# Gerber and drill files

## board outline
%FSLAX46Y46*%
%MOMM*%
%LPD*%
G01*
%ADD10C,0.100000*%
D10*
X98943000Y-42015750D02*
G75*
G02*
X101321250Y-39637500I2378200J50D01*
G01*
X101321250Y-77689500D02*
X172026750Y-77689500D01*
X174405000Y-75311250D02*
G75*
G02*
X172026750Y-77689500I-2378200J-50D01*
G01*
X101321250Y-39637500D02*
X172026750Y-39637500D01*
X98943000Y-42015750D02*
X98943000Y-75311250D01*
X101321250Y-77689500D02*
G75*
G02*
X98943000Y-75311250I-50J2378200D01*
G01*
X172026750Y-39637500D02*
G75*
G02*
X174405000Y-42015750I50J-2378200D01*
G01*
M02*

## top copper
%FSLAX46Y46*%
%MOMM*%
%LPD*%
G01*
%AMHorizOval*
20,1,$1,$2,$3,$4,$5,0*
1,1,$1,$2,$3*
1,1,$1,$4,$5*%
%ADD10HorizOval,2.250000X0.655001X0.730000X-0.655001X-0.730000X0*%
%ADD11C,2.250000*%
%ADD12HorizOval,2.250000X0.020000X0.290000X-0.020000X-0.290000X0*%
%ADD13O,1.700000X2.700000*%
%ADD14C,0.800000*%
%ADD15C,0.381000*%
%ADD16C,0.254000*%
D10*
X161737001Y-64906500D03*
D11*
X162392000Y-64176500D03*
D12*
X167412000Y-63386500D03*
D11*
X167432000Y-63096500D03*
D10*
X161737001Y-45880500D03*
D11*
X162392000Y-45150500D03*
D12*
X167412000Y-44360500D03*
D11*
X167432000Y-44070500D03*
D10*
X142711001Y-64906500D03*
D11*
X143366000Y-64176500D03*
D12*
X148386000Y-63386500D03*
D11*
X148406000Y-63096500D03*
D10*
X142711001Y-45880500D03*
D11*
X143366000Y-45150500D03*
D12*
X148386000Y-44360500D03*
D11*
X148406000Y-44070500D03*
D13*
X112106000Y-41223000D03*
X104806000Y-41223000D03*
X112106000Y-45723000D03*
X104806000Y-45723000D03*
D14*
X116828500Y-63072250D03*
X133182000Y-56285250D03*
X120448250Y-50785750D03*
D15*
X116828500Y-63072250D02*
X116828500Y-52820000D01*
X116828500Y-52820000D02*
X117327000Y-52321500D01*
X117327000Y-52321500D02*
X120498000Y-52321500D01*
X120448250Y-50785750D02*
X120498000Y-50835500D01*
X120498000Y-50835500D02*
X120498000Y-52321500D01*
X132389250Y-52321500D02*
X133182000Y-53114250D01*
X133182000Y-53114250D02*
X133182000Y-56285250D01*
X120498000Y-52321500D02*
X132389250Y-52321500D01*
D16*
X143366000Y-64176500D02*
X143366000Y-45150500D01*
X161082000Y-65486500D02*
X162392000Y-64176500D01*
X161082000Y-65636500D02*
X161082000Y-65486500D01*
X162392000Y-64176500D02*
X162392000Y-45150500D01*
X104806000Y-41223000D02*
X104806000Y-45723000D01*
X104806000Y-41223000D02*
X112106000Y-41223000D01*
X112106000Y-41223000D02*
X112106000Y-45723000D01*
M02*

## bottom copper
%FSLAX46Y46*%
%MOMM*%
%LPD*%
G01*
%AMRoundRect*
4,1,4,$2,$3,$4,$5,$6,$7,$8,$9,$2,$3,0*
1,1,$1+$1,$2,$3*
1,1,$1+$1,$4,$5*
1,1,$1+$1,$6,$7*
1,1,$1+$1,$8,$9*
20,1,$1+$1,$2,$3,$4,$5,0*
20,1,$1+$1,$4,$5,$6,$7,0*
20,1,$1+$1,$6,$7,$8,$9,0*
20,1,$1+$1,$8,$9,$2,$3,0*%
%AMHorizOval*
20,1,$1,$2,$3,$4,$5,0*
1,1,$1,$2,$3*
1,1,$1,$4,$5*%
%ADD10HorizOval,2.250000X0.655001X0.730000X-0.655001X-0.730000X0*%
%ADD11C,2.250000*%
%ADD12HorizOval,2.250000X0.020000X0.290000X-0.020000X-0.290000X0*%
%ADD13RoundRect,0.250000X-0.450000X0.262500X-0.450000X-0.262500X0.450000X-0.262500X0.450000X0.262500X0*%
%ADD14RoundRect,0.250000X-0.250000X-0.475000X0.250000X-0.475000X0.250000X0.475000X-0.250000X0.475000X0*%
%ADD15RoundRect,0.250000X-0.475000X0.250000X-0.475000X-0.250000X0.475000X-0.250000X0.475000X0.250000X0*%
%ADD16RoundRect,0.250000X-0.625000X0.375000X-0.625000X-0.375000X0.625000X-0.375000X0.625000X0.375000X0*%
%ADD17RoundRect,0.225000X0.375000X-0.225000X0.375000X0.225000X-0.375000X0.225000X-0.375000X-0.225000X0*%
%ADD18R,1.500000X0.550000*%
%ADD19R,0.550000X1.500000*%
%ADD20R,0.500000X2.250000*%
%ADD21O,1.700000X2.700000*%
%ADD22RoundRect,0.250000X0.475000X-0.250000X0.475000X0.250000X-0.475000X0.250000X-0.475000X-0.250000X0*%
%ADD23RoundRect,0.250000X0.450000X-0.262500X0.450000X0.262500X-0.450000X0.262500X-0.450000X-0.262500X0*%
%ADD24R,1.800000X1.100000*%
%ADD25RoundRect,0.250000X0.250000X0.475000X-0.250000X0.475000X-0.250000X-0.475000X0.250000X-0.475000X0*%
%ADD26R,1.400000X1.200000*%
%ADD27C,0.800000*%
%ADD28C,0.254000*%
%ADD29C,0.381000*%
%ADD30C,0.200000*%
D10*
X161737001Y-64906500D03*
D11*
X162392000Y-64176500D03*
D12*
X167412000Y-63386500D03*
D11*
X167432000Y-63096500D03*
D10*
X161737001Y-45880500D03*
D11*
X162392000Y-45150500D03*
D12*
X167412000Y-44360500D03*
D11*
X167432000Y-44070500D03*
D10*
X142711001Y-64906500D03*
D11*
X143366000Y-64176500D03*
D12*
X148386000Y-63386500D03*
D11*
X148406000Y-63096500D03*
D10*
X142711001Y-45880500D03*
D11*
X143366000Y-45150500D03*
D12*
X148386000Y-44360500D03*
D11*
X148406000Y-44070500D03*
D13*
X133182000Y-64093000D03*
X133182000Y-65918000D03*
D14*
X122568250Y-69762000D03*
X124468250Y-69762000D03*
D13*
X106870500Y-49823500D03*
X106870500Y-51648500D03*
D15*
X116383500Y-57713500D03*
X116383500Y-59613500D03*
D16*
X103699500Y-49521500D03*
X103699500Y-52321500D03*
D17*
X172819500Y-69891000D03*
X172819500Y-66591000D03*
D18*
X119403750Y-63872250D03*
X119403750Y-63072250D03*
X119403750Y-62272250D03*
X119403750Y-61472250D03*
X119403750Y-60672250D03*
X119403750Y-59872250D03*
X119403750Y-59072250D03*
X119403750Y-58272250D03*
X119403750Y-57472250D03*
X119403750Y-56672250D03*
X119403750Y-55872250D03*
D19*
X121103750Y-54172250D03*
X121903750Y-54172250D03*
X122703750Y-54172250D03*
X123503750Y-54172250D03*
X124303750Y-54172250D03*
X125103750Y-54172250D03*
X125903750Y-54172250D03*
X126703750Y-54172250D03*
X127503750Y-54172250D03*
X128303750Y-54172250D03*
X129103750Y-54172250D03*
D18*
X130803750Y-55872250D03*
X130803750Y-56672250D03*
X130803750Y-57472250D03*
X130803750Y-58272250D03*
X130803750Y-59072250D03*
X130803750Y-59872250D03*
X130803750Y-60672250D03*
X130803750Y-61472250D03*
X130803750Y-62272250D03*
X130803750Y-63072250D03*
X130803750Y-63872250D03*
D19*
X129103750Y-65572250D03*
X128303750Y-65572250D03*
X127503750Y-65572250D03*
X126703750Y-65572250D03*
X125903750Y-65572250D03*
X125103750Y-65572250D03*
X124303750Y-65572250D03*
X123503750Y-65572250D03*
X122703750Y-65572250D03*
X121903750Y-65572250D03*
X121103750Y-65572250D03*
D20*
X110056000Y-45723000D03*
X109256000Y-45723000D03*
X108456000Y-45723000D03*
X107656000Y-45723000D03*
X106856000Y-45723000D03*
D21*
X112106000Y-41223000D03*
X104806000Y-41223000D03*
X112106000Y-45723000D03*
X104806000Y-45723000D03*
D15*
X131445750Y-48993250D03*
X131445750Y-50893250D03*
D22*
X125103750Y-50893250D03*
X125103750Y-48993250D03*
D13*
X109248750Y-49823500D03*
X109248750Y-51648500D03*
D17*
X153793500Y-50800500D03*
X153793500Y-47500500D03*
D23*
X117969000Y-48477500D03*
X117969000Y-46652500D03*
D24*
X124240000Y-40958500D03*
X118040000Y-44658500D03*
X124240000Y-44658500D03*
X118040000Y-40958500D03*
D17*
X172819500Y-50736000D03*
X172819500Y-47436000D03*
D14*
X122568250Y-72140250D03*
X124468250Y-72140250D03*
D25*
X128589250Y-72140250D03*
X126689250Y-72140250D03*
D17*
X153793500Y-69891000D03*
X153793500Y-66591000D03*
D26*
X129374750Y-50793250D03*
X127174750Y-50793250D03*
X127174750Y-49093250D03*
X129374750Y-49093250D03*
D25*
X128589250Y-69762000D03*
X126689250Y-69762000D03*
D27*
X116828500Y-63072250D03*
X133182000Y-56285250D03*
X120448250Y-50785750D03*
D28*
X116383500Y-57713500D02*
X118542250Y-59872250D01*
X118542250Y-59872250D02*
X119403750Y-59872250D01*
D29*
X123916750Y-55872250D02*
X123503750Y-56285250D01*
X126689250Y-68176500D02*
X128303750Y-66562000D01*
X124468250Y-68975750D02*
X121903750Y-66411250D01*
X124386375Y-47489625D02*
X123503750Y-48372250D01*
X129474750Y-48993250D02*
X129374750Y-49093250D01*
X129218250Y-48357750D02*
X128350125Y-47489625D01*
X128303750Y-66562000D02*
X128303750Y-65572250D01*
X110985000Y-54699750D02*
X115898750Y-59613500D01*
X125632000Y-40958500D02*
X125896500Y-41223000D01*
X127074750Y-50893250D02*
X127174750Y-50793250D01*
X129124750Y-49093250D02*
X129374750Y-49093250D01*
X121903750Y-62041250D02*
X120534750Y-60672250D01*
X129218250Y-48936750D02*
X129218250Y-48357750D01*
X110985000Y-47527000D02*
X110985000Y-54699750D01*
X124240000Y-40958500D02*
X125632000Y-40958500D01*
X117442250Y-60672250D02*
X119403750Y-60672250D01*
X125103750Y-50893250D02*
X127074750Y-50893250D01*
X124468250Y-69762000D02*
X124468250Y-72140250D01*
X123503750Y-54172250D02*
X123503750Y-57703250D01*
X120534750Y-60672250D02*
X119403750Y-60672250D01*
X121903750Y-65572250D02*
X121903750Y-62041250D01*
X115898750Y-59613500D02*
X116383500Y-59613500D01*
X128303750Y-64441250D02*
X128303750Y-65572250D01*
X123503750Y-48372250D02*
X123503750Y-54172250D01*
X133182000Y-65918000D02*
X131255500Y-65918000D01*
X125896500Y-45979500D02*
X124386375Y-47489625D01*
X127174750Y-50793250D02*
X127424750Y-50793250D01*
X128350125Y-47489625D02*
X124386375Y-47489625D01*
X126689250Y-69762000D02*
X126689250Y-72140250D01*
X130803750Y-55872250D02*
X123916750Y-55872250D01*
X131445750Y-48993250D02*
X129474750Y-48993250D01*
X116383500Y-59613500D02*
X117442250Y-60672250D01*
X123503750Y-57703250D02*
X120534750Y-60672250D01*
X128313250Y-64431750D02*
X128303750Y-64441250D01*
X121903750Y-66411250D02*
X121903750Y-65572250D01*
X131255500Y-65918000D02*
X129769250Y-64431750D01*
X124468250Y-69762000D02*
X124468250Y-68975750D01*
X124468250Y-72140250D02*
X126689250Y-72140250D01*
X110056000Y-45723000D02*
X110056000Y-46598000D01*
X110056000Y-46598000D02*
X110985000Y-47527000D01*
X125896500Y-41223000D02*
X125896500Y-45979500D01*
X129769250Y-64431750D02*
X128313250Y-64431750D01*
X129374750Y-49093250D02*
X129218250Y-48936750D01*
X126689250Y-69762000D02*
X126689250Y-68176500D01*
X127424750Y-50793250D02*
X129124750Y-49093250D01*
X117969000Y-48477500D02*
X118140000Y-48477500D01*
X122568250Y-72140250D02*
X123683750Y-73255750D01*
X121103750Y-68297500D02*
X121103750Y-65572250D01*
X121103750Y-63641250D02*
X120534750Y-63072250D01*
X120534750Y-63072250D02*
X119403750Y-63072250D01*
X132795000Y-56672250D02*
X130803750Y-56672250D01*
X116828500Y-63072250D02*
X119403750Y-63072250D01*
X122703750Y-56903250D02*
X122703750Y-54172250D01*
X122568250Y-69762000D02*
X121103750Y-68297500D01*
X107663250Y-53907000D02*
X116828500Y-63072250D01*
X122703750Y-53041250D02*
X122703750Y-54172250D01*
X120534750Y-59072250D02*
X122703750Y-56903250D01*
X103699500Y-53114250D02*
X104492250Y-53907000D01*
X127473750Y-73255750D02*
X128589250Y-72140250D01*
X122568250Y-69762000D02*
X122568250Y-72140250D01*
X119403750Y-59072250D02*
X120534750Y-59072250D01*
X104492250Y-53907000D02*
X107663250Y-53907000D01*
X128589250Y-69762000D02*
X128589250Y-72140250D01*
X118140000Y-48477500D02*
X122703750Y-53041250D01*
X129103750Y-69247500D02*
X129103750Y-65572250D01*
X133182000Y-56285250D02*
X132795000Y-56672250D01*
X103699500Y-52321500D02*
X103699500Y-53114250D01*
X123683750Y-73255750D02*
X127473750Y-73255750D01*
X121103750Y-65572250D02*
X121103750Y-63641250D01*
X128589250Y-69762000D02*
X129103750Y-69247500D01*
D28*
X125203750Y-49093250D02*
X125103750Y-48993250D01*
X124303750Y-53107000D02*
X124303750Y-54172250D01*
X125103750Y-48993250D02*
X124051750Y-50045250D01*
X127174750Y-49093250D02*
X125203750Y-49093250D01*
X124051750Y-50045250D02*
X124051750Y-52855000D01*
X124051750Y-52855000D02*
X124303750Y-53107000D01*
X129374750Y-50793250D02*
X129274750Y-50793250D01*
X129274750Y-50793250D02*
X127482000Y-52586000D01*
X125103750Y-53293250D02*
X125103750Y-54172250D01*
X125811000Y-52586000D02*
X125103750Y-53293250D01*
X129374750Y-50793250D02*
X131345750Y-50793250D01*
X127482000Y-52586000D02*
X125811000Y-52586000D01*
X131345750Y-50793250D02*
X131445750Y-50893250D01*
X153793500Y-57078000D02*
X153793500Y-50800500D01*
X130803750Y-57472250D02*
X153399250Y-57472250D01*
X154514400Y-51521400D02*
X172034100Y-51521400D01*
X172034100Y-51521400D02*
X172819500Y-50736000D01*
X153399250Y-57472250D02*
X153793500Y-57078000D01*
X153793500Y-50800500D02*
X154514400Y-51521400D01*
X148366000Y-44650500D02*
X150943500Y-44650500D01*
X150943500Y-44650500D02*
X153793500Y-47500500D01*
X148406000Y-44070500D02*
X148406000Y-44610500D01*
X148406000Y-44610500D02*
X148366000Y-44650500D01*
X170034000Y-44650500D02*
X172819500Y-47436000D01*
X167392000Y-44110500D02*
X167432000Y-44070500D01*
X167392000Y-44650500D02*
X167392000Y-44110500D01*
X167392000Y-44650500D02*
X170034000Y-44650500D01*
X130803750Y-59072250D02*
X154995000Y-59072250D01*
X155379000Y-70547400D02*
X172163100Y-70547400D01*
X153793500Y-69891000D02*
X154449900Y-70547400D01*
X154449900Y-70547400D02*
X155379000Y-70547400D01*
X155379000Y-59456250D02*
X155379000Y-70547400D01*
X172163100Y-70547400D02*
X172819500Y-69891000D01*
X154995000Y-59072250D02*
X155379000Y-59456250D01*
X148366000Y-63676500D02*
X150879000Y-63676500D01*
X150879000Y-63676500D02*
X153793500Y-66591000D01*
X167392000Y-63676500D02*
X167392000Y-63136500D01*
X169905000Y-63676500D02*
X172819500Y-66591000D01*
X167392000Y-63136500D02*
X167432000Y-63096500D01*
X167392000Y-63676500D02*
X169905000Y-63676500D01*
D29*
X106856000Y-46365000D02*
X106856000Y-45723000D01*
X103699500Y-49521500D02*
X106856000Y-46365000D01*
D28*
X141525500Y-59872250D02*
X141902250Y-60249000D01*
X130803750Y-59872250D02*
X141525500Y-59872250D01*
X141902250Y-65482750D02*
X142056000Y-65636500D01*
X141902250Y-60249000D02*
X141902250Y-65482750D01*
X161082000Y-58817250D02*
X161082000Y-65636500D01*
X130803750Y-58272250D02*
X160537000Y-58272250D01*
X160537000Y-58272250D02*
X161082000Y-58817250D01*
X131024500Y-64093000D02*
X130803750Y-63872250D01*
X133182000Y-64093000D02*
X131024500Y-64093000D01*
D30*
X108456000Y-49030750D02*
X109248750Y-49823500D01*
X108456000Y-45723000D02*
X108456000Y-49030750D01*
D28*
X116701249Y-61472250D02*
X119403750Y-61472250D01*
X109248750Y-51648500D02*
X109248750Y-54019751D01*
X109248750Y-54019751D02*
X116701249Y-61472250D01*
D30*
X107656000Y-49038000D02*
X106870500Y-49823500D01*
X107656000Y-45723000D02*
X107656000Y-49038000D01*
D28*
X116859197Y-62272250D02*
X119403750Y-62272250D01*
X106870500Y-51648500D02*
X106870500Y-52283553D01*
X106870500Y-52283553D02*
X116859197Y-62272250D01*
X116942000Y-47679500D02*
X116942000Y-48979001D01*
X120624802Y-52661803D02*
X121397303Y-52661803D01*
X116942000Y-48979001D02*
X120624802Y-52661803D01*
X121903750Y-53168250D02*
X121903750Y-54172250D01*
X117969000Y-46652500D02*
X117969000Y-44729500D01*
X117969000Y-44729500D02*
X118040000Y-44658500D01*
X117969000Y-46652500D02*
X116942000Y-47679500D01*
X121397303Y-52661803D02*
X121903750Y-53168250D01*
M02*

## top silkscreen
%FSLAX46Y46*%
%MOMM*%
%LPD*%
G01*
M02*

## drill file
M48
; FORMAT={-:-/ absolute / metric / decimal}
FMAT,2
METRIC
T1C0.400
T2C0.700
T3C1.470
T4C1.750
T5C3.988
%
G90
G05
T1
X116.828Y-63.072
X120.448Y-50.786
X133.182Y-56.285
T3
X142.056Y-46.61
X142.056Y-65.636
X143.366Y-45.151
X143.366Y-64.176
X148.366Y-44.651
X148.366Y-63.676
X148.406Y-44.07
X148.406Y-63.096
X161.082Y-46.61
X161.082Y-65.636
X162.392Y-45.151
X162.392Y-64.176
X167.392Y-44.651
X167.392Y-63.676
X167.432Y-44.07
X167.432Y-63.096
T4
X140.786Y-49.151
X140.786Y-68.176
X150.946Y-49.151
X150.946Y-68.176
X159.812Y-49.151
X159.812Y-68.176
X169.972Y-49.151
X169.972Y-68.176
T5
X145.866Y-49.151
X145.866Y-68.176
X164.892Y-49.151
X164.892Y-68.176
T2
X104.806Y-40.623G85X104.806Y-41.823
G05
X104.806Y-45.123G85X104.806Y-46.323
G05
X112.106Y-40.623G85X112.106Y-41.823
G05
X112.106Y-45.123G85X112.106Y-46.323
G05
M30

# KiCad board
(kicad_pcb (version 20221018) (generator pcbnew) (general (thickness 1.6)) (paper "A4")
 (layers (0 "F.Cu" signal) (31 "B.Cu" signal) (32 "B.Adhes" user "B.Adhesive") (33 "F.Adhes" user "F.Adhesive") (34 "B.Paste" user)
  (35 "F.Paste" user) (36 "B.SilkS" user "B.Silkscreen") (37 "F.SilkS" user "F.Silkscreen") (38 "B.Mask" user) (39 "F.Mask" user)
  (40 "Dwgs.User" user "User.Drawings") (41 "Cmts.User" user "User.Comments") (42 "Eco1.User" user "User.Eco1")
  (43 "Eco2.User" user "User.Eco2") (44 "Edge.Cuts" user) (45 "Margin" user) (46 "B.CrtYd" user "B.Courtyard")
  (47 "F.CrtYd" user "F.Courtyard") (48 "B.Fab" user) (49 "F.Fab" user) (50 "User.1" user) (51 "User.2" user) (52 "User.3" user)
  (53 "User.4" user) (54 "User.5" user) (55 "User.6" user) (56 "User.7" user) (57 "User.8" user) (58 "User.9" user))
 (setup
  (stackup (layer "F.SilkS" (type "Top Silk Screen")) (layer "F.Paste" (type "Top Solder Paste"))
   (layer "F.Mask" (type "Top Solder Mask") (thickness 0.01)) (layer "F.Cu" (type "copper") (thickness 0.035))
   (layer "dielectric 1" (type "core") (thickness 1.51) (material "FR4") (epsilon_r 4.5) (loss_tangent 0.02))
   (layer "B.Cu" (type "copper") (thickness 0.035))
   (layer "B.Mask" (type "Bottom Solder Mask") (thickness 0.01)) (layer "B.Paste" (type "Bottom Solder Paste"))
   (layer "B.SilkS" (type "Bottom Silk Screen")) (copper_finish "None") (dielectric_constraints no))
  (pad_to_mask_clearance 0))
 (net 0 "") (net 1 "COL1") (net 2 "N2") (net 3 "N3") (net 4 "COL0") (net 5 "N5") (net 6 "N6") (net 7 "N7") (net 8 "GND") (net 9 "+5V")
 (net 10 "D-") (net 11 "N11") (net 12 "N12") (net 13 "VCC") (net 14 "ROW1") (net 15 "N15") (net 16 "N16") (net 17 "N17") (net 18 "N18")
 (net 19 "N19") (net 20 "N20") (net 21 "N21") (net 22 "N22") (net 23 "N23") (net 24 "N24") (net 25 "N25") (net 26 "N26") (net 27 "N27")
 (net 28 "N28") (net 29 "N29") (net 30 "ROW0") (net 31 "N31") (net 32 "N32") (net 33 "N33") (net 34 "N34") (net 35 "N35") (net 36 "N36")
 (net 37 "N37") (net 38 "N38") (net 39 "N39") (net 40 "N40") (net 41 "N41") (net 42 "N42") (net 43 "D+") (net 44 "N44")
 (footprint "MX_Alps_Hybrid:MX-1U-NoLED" (layer "F.Cu") (at 164.892 68.1765)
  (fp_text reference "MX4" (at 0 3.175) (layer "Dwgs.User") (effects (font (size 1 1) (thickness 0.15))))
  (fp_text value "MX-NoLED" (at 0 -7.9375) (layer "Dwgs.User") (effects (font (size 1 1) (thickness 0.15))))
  (pad "" np_thru_hole circle (at -5.08 0 48.0996) (size 1.75 1.75) (drill 1.75) (layers "*.Cu" "*.Mask"))
  (pad "" np_thru_hole circle (at 0 0) (size 3.9878 3.9878) (drill 3.9878) (layers "*.Cu" "*.Mask"))
  (pad "" np_thru_hole circle (at 5.08 0 48.0996) (size 1.75 1.75) (drill 1.75) (layers "*.Cu" "*.Mask"))
  (pad "1" thru_hole oval (at -3.81 -2.54 48.0996) (size 4.211556 2.25) (drill 1.47 (offset 0.980778 0)) (layers "*.Cu" "B.Mask")
   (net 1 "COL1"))
  (pad "1" thru_hole circle (at -2.5 -4) (size 2.25 2.25) (drill 1.47) (layers "*.Cu" "B.Mask") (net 1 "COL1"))
  (pad "2" thru_hole oval (at 2.5 -4.5 86.0548) (size 2.831378 2.25) (drill 1.47 (offset 0.290689 0)) (layers "*.Cu" "B.Mask") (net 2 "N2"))
  (pad "2" thru_hole circle (at 2.54 -5.08) (size 2.25 2.25) (drill 1.47) (layers "*.Cu" "B.Mask") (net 2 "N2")))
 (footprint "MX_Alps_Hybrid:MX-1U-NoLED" (layer "F.Cu") (at 164.892 49.1505)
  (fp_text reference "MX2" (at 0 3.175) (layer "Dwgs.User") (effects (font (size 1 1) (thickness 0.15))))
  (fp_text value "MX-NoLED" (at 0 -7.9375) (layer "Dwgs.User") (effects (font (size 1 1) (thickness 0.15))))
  (pad "" np_thru_hole circle (at -5.08 0 48.0996) (size 1.75 1.75) (drill 1.75) (layers "*.Cu" "*.Mask"))
  (pad "" np_thru_hole circle (at 0 0) (size 3.9878 3.9878) (drill 3.9878) (layers "*.Cu" "*.Mask"))
  (pad "" np_thru_hole circle (at 5.08 0 48.0996) (size 1.75 1.75) (drill 1.75) (layers "*.Cu" "*.Mask"))
  (pad "1" thru_hole oval (at -3.81 -2.54 48.0996) (size 4.211556 2.25) (drill 1.47 (offset 0.980778 0)) (layers "*.Cu" "B.Mask")
   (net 1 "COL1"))
  (pad "1" thru_hole circle (at -2.5 -4) (size 2.25 2.25) (drill 1.47) (layers "*.Cu" "B.Mask") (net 1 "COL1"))
  (pad "2" thru_hole oval (at 2.5 -4.5 86.0548) (size 2.831378 2.25) (drill 1.47 (offset 0.290689 0)) (layers "*.Cu" "B.Mask") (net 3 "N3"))
  (pad "2" thru_hole circle (at 2.54 -5.08) (size 2.25 2.25) (drill 1.47) (layers "*.Cu" "B.Mask") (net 3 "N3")))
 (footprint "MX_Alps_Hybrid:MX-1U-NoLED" (layer "F.Cu") (at 145.866 68.1765)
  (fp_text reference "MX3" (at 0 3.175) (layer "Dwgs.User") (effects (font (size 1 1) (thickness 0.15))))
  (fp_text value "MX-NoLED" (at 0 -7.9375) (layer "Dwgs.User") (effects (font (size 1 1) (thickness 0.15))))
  (pad "" np_thru_hole circle (at -5.08 0 48.0996) (size 1.75 1.75) (drill 1.75) (layers "*.Cu" "*.Mask"))
  (pad "" np_thru_hole circle (at 0 0) (size 3.9878 3.9878) (drill 3.9878) (layers "*.Cu" "*.Mask"))
  (pad "" np_thru_hole circle (at 5.08 0 48.0996) (size 1.75 1.75) (drill 1.75) (layers "*.Cu" "*.Mask"))
  (pad "1" thru_hole oval (at -3.81 -2.54 48.0996) (size 4.211556 2.25) (drill 1.47 (offset 0.980778 0)) (layers "*.Cu" "B.Mask")
   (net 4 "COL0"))
  (pad "1" thru_hole circle (at -2.5 -4) (size 2.25 2.25) (drill 1.47) (layers "*.Cu" "B.Mask") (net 4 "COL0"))
  (pad "2" thru_hole oval (at 2.5 -4.5 86.0548) (size 2.831378 2.25) (drill 1.47 (offset 0.290689 0)) (layers "*.Cu" "B.Mask") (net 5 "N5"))
  (pad "2" thru_hole circle (at 2.54 -5.08) (size 2.25 2.25) (drill 1.47) (layers "*.Cu" "B.Mask") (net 5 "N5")))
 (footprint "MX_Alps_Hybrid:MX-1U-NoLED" (layer "F.Cu") (at 145.866 49.1505)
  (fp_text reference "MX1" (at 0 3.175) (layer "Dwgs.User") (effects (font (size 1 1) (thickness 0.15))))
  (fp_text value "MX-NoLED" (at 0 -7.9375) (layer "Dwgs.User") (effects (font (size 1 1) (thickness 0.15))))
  (pad "" np_thru_hole circle (at -5.08 0 48.0996) (size 1.75 1.75) (drill 1.75) (layers "*.Cu" "*.Mask"))
  (pad "" np_thru_hole circle (at 0 0) (size 3.9878 3.9878) (drill 3.9878) (layers "*.Cu" "*.Mask"))
  (pad "" np_thru_hole circle (at 5.08 0 48.0996) (size 1.75 1.75) (drill 1.75) (layers "*.Cu" "*.Mask"))
  (pad "1" thru_hole oval (at -3.81 -2.54 48.0996) (size 4.211556 2.25) (drill 1.47 (offset 0.980778 0)) (layers "*.Cu" "B.Mask")
   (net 4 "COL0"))
  (pad "1" thru_hole circle (at -2.5 -4) (size 2.25 2.25) (drill 1.47) (layers "*.Cu" "B.Mask") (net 4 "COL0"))
  (pad "2" thru_hole oval (at 2.5 -4.5 86.0548) (size 2.831378 2.25) (drill 1.47 (offset 0.290689 0)) (layers "*.Cu" "B.Mask") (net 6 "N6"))
  (pad "2" thru_hole circle (at 2.54 -5.08) (size 2.25 2.25) (drill 1.47) (layers "*.Cu" "B.Mask") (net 6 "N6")))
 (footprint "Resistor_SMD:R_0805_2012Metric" (layer "B.Cu") (at 133.182 65.0055 -90)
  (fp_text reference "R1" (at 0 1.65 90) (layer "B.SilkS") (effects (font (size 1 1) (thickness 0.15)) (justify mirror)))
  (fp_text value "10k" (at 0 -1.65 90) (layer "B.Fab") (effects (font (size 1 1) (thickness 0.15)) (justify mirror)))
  (pad "1" smd roundrect (at -0.9125 0 270) (size 1.025 1.4) (layers "B.Cu" "B.Paste" "B.Mask") (roundrect_rratio 0.243902) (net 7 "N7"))
  (pad "2" smd roundrect (at 0.9125 0 270) (size 1.025 1.4) (layers "B.Cu" "B.Paste" "B.Mask") (roundrect_rratio 0.243902) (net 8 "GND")))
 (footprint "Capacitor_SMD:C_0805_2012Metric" (layer "B.Cu") (at 123.51825 69.762)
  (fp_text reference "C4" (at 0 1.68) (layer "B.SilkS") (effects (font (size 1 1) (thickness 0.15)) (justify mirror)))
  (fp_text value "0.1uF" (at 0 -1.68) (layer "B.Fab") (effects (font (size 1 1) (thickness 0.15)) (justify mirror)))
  (pad "1" smd roundrect (at -0.95 0) (size 1 1.45) (layers "B.Cu" "B.Paste" "B.Mask") (roundrect_rratio 0.25) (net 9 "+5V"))
  (pad "2" smd roundrect (at 0.95 0) (size 1 1.45) (layers "B.Cu" "B.Paste" "B.Mask") (roundrect_rratio 0.25) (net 8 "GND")))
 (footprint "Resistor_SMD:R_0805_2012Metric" (layer "B.Cu") (at 106.8705 50.736 -90)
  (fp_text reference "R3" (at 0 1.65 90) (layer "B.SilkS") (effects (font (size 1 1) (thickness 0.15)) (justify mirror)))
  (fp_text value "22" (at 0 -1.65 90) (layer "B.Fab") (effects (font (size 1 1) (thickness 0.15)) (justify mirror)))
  (pad "1" smd roundrect (at -0.9125 0 270) (size 1.025 1.4) (layers "B.Cu" "B.Paste" "B.Mask") (roundrect_rratio 0.243902) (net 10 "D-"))
  (pad "2" smd roundrect (at 0.9125 0 270) (size 1.025 1.4) (layers "B.Cu" "B.Paste" "B.Mask") (roundrect_rratio 0.243902) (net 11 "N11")))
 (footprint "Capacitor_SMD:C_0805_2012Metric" (layer "B.Cu") (at 116.3835 58.6635 -90)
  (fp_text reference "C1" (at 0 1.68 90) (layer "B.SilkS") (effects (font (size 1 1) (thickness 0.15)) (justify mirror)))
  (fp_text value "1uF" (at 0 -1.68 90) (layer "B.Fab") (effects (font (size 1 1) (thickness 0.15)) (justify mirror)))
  (pad "1" smd roundrect (at -0.95 0 270) (size 1 1.45) (layers "B.Cu" "B.Paste" "B.Mask") (roundrect_rratio 0.25) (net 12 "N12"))
  (pad "2" smd roundrect (at 0.95 0 270) (size 1 1.45) (layers "B.Cu" "B.Paste" "B.Mask") (roundrect_rratio 0.25) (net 8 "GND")))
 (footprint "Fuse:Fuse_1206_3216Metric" (layer "B.Cu") (at 103.6995 50.9215 -90)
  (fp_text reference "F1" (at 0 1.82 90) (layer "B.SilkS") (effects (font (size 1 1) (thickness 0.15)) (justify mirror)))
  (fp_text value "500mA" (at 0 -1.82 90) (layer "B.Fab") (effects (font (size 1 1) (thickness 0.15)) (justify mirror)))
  (pad "1" smd roundrect (at -1.4 0 270) (size 1.25 1.75) (layers "B.Cu" "B.Paste" "B.Mask") (roundrect_rratio 0.2) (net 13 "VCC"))
  (pad "2" smd roundrect (at 1.4 0 270) (size 1.25 1.75) (layers "B.Cu" "B.Paste" "B.Mask") (roundrect_rratio 0.2) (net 9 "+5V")))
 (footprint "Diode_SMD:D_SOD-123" (layer "B.Cu") (at 172.8195 68.241 90)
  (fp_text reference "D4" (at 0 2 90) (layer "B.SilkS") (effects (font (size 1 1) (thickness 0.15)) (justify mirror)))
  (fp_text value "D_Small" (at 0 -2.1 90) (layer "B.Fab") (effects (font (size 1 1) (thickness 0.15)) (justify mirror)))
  (pad "1" smd roundrect (at -1.65 0 90) (size 0.9 1.2) (layers "B.Cu" "B.Paste" "B.Mask") (roundrect_rratio 0.25) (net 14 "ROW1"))
  (pad "2" smd roundrect (at 1.65 0 90) (size 0.9 1.2) (layers "B.Cu" "B.Paste" "B.Mask") (roundrect_rratio 0.25) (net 2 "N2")))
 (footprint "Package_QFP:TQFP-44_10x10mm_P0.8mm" (layer "B.Cu") (at 125.10375 59.87225)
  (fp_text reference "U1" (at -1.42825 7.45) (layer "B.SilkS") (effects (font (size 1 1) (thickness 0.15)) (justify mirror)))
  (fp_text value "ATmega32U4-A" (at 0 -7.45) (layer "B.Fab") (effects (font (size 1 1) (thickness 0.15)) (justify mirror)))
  (pad "1" smd rect (at -5.7 4) (size 1.5 0.55) (layers "B.Cu" "B.Paste" "B.Mask") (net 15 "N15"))
  (pad "2" smd rect (at -5.7 3.2) (size 1.5 0.55) (layers "B.Cu" "B.Paste" "B.Mask") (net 9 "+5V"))
  (pad "3" smd rect (at -5.7 2.4) (size 1.5 0.55) (layers "B.Cu" "B.Paste" "B.Mask") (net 11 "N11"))
  (pad "4" smd rect (at -5.7 1.6) (size 1.5 0.55) (layers "B.Cu" "B.Paste" "B.Mask") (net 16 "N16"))
  (pad "5" smd rect (at -5.7 0.8) (size 1.5 0.55) (layers "B.Cu" "B.Paste" "B.Mask") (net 8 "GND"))
  (pad "6" smd rect (at -5.7 0) (size 1.5 0.55) (layers "B.Cu" "B.Paste" "B.Mask") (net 12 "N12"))
  (pad "7" smd rect (at -5.7 -0.8) (size 1.5 0.55) (layers "B.Cu" "B.Paste" "B.Mask") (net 9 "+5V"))
  (pad "8" smd rect (at -5.7 -1.6) (size 1.5 0.55) (layers "B.Cu" "B.Paste" "B.Mask") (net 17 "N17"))
  (pad "9" smd rect (at -5.7 -2.4) (size 1.5 0.55) (layers "B.Cu" "B.Paste" "B.Mask") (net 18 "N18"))
  (pad "10" smd rect (at -5.7 -3.2) (size 1.5 0.55) (layers "B.Cu" "B.Paste" "B.Mask") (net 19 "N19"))
  (pad "11" smd rect (at -5.7 -4) (size 1.5 0.55) (layers "B.Cu" "B.Paste" "B.Mask") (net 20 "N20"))
  (pad "12" smd rect (at -4 -5.7 270) (size 1.5 0.55) (layers "B.Cu" "B.Paste" "B.Mask") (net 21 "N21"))
  (pad "13" smd rect (at -3.2 -5.7 270) (size 1.5 0.55) (layers "B.Cu" "B.Paste" "B.Mask") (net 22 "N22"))
  (pad "14" smd rect (at -2.4 -5.7 270) (size 1.5 0.55) (layers "B.Cu" "B.Paste" "B.Mask") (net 9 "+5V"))
  (pad "15" smd rect (at -1.6 -5.7 270) (size 1.5 0.55) (layers "B.Cu" "B.Paste" "B.Mask") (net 8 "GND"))
  (pad "16" smd rect (at -0.8 -5.7 270) (size 1.5 0.55) (layers "B.Cu" "B.Paste" "B.Mask") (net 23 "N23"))
  (pad "17" smd rect (at 0 -5.7 270) (size 1.5 0.55) (layers "B.Cu" "B.Paste" "B.Mask") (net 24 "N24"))
  (pad "18" smd rect (at 0.8 -5.7 270) (size 1.5 0.55) (layers "B.Cu" "B.Paste" "B.Mask") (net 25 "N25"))
  (pad "19" smd rect (at 1.6 -5.7 270) (size 1.5 0.55) (layers "B.Cu" "B.Paste" "B.Mask") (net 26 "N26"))
  (pad "20" smd rect (at 2.4 -5.7 270) (size 1.5 0.55) (layers "B.Cu" "B.Paste" "B.Mask") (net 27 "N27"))
  (pad "21" smd rect (at 3.2 -5.7 270) (size 1.5 0.55) (layers "B.Cu" "B.Paste" "B.Mask") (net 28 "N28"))
  (pad "22" smd rect (at 4 -5.7 270) (size 1.5 0.55) (layers "B.Cu" "B.Paste" "B.Mask") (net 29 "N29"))
  (pad "23" smd rect (at 5.7 -4) (size 1.5 0.55) (layers "B.Cu" "B.Paste" "B.Mask") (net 8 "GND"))
  (pad "24" smd rect (at 5.7 -3.2) (size 1.5 0.55) (layers "B.Cu" "B.Paste" "B.Mask") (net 9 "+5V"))
  (pad "25" smd rect (at 5.7 -2.4) (size 1.5 0.55) (layers "B.Cu" "B.Paste" "B.Mask") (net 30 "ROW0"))
  (pad "26" smd rect (at 5.7 -1.6) (size 1.5 0.55) (layers "B.Cu" "B.Paste" "B.Mask") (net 1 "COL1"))
  (pad "27" smd rect (at 5.7 -0.8) (size 1.5 0.55) (layers "B.Cu" "B.Paste" "B.Mask") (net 14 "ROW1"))
  (pad "28" smd rect (at 5.7 0) (size 1.5 0.55) (layers "B.Cu" "B.Paste" "B.Mask") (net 4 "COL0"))
  (pad "29" smd rect (at 5.7 0.8) (size 1.5 0.55) (layers "B.Cu" "B.Paste" "B.Mask") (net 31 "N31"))
  (pad "30" smd rect (at 5.7 1.6) (size 1.5 0.55) (layers "B.Cu" "B.Paste" "B.Mask") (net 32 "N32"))
  (pad "31" smd rect (at 5.7 2.4) (size 1.5 0.55) (layers "B.Cu" "B.Paste" "B.Mask") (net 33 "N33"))
  (pad "32" smd rect (at 5.7 3.2) (size 1.5 0.55) (layers "B.Cu" "B.Paste" "B.Mask") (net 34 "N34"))
  (pad "33" smd rect (at 5.7 4) (size 1.5 0.55) (layers "B.Cu" "B.Paste" "B.Mask") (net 7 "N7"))
  (pad "34" smd rect (at 4 5.7 270) (size 1.5 0.55) (layers "B.Cu" "B.Paste" "B.Mask") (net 9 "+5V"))
  (pad "35" smd rect (at 3.2 5.7 270) (size 1.5 0.55) (layers "B.Cu" "B.Paste" "B.Mask") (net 8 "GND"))
  (pad "36" smd rect (at 2.4 5.7 270) (size 1.5 0.55) (layers "B.Cu" "B.Paste" "B.Mask") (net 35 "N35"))
  (pad "37" smd rect (at 1.6 5.7 270) (size 1.5 0.55) (layers "B.Cu" "B.Paste" "B.Mask") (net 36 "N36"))
  (pad "38" smd rect (at 0.8 5.7 270) (size 1.5 0.55) (layers "B.Cu" "B.Paste" "B.Mask") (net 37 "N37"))
  (pad "39" smd rect (at 0 5.7 270) (size 1.5 0.55) (layers "B.Cu" "B.Paste" "B.Mask") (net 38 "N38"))
  (pad "40" smd rect (at -0.8 5.7 270) (size 1.5 0.55) (layers "B.Cu" "B.Paste" "B.Mask") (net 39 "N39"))
  (pad "41" smd rect (at -1.6 5.7 270) (size 1.5 0.55) (layers "B.Cu" "B.Paste" "B.Mask") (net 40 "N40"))
  (pad "42" smd rect (at -2.4 5.7 270) (size 1.5 0.55) (layers "B.Cu" "B.Paste" "B.Mask") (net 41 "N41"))
  (pad "43" smd rect (at -3.2 5.7 270) (size 1.5 0.55) (layers "B.Cu" "B.Paste" "B.Mask") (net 8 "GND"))
  (pad "44" smd rect (at -4 5.7 270) (size 1.5 0.55) (layers "B.Cu" "B.Paste" "B.Mask") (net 9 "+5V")))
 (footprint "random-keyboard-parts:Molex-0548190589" (layer "B.Cu") (at 108.456 41.223 -90)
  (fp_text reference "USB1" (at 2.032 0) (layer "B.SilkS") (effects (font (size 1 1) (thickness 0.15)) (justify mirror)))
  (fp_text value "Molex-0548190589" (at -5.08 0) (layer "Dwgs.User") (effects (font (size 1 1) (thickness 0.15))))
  (pad "1" smd rect (at 4.5 -1.6 270) (size 2.25 0.5) (layers "B.Cu" "B.Paste" "B.Mask") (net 8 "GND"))
  (pad "2" smd rect (at 4.5 -0.8 270) (size 2.25 0.5) (layers "B.Cu" "B.Paste" "B.Mask") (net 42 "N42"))
  (pad "3" smd rect (at 4.5 0 270) (size 2.25 0.5) (layers "B.Cu" "B.Paste" "B.Mask") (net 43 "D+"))
  (pad "4" smd rect (at 4.5 0.8 270) (size 2.25 0.5) (layers "B.Cu" "B.Paste" "B.Mask") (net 10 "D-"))
  (pad "5" smd rect (at 4.5 1.6 270) (size 2.25 0.5) (layers "B.Cu" "B.Paste" "B.Mask") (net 13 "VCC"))
  (pad "6" thru_hole oval (at 0 -3.65 270) (size 2.7 1.7) (drill oval 1.9 0.7) (layers "*.Cu" "*.Mask") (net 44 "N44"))
  (pad "6" thru_hole oval (at 0 3.65 270) (size 2.7 1.7) (drill oval 1.9 0.7) (layers "*.Cu" "*.Mask") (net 44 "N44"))
  (pad "6" thru_hole oval (at 4.5 -3.65 270) (size 2.7 1.7) (drill oval 1.9 0.7) (layers "*.Cu" "*.Mask") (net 44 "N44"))
  (pad "6" thru_hole oval (at 4.5 3.65 270) (size 2.7 1.7) (drill oval 1.9 0.7) (layers "*.Cu" "*.Mask") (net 44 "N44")))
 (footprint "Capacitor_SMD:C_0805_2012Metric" (layer "B.Cu") (at 131.44575 49.94325 -90)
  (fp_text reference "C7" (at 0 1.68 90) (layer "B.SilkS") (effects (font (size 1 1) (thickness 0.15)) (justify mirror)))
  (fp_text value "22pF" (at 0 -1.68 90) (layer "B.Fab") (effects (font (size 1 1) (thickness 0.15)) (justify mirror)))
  (pad "1" smd roundrect (at -0.95 0 270) (size 1 1.45) (layers "B.Cu" "B.Paste" "B.Mask") (roundrect_rratio 0.25) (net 8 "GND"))
  (pad "2" smd roundrect (at 0.95 0 270) (size 1 1.45) (layers "B.Cu" "B.Paste" "B.Mask") (roundrect_rratio 0.25) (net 24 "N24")))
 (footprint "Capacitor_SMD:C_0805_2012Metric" (layer "B.Cu") (at 125.10375 49.94325 90)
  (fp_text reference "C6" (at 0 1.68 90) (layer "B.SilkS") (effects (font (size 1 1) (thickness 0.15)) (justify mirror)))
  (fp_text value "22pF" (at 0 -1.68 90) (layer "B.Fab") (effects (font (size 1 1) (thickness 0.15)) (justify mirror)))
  (pad "1" smd roundrect (at -0.95 0 90) (size 1 1.45) (layers "B.Cu" "B.Paste" "B.Mask") (roundrect_rratio 0.25) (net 8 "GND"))
  (pad "2" smd roundrect (at 0.95 0 90) (size 1 1.45) (layers "B.Cu" "B.Paste" "B.Mask") (roundrect_rratio 0.25) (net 23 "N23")))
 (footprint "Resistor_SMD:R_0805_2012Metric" (layer "B.Cu") (at 109.24875 50.736 -90)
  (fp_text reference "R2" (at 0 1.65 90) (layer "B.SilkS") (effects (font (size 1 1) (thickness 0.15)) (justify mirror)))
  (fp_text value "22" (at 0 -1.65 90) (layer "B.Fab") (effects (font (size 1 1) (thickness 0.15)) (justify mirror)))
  (pad "1" smd roundrect (at -0.9125 0 270) (size 1.025 1.4) (layers "B.Cu" "B.Paste" "B.Mask") (roundrect_rratio 0.243902) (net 43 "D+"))
  (pad "2" smd roundrect (at 0.9125 0 270) (size 1.025 1.4) (layers "B.Cu" "B.Paste" "B.Mask") (roundrect_rratio 0.243902) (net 16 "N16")))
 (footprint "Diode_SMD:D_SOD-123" (layer "B.Cu") (at 153.7935 49.1505 90)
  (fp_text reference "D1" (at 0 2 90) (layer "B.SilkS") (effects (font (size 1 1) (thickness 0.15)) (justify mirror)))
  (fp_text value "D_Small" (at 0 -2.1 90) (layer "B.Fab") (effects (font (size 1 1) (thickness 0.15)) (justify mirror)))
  (pad "1" smd roundrect (at -1.65 0 90) (size 0.9 1.2) (layers "B.Cu" "B.Paste" "B.Mask") (roundrect_rratio 0.25) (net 30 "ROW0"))
  (pad "2" smd roundrect (at 1.65 0 90) (size 0.9 1.2) (layers "B.Cu" "B.Paste" "B.Mask") (roundrect_rratio 0.25) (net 6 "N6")))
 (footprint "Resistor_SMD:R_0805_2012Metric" (layer "B.Cu") (at 117.969 47.565 90)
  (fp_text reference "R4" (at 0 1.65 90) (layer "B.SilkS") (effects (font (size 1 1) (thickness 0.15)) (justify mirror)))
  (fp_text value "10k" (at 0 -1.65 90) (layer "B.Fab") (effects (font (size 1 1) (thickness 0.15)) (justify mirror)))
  (pad "1" smd roundrect (at -0.9125 0 90) (size 1.025 1.4) (layers "B.Cu" "B.Paste" "B.Mask") (roundrect_rratio 0.243902) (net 9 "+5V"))
  (pad "2" smd roundrect (at 0.9125 0 90) (size 1.025 1.4) (layers "B.Cu" "B.Paste" "B.Mask") (roundrect_rratio 0.243902) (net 22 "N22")))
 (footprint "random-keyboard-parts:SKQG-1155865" (layer "B.Cu") (at 121.14 42.8085)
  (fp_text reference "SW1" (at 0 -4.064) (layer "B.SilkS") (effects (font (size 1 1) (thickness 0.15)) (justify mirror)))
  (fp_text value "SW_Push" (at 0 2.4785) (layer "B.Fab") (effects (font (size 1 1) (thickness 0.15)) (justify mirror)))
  (pad "1" smd rect (at 3.1 -1.85) (size 1.8 1.1) (layers "B.Cu" "B.Paste" "B.Mask") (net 8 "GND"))
  (pad "2" smd rect (at -3.1 1.85) (size 1.8 1.1) (layers "B.Cu" "B.Paste" "B.Mask") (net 22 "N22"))
  (pad "3" smd rect (at 3.1 1.85) (size 1.8 1.1) (layers "B.Cu" "B.Paste" "B.Mask"))
  (pad "4" smd rect (at -3.1 -1.85) (size 1.8 1.1) (layers "B.Cu" "B.Paste" "B.Mask")))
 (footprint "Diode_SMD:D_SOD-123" (layer "B.Cu") (at 172.8195 49.086 90)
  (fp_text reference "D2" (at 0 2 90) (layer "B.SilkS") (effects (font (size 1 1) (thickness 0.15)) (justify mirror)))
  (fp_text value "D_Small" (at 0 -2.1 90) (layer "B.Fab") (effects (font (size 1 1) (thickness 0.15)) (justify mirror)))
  (pad "1" smd roundrect (at -1.65 0 90) (size 0.9 1.2) (layers "B.Cu" "B.Paste" "B.Mask") (roundrect_rratio 0.25) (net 30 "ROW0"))
  (pad "2" smd roundrect (at 1.65 0 90) (size 0.9 1.2) (layers "B.Cu" "B.Paste" "B.Mask") (roundrect_rratio 0.25) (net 3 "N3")))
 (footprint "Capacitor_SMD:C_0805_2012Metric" (layer "B.Cu") (at 123.51825 72.14025)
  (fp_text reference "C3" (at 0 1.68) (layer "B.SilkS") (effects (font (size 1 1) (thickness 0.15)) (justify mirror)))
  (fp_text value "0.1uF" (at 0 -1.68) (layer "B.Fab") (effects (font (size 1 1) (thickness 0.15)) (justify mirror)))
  (pad "1" smd roundrect (at -0.95 0) (size 1 1.45) (layers "B.Cu" "B.Paste" "B.Mask") (roundrect_rratio 0.25) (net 9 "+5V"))
  (pad "2" smd roundrect (at 0.95 0) (size 1 1.45) (layers "B.Cu" "B.Paste" "B.Mask") (roundrect_rratio 0.25) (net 8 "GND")))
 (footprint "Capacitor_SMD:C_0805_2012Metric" (layer "B.Cu") (at 127.63925 72.14025 180)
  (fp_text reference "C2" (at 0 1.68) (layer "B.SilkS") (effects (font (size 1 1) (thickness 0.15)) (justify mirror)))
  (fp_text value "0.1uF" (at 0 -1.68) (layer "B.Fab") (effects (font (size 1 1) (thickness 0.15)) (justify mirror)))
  (pad "1" smd roundrect (at -0.95 0 180) (size 1 1.45) (layers "B.Cu" "B.Paste" "B.Mask") (roundrect_rratio 0.25) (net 9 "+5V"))
  (pad "2" smd roundrect (at 0.95 0 180) (size 1 1.45) (layers "B.Cu" "B.Paste" "B.Mask") (roundrect_rratio 0.25) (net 8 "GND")))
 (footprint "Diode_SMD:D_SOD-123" (layer "B.Cu") (at 153.7935 68.241 90)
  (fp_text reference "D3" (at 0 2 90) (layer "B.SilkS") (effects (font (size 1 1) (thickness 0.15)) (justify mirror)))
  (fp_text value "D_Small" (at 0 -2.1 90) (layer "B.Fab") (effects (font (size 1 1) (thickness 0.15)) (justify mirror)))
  (pad "1" smd roundrect (at -1.65 0 90) (size 0.9 1.2) (layers "B.Cu" "B.Paste" "B.Mask") (roundrect_rratio 0.25) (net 14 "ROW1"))
  (pad "2" smd roundrect (at 1.65 0 90) (size 0.9 1.2) (layers "B.Cu" "B.Paste" "B.Mask") (roundrect_rratio 0.25) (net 5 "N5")))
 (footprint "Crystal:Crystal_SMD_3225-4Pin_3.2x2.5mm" (layer "B.Cu") (at 128.27475 49.94325 180)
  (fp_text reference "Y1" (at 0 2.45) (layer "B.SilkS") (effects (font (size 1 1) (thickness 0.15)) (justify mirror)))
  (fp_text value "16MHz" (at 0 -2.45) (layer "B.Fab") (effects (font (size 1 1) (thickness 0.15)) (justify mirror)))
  (pad "1" smd rect (at -1.1 -0.85 180) (size 1.4 1.2) (layers "B.Cu" "B.Paste" "B.Mask") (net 24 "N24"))
  (pad "2" smd rect (at 1.1 -0.85 180) (size 1.4 1.2) (layers "B.Cu" "B.Paste" "B.Mask") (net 8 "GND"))
  (pad "3" smd rect (at 1.1 0.85 180) (size 1.4 1.2) (layers "B.Cu" "B.Paste" "B.Mask") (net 23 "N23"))
  (pad "4" smd rect (at -1.1 0.85 180) (size 1.4 1.2) (layers "B.Cu" "B.Paste" "B.Mask") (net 8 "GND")))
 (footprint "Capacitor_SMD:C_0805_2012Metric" (layer "B.Cu") (at 127.63925 69.762 180)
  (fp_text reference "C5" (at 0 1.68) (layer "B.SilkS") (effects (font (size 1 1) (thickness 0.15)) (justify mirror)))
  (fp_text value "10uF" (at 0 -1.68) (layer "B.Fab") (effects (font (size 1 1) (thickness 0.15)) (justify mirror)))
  (pad "1" smd roundrect (at -0.95 0 180) (size 1 1.45) (layers "B.Cu" "B.Paste" "B.Mask") (roundrect_rratio 0.25) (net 9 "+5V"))
  (pad "2" smd roundrect (at 0.95 0 180) (size 1 1.45) (layers "B.Cu" "B.Paste" "B.Mask") (roundrect_rratio 0.25) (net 8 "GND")))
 (gr_arc (start 98.943 42.01575) (mid 99.639573 40.334073) (end 101.32125 39.6375) (stroke (width 0.1) (type default)) (layer "Edge.Cuts"))
 (gr_line (start 101.32125 77.6895) (end 172.02675 77.6895) (stroke (width 0.1) (type default)) (layer "Edge.Cuts"))
 (gr_arc (start 174.405 75.31125) (mid 173.708427 76.992927) (end 172.02675 77.6895) (stroke (width 0.1) (type default)) (layer "Edge.Cuts"))
 (gr_line (start 101.32125 39.6375) (end 172.02675 39.6375) (stroke (width 0.1) (type default)) (layer "Edge.Cuts"))
 (gr_line (start 98.943 42.01575) (end 98.943 75.31125) (stroke (width 0.1) (type default)) (layer "Edge.Cuts"))
 (gr_arc (start 101.32125 77.6895) (mid 99.639573 76.992927) (end 98.943 75.31125) (stroke (width 0.1) (type default)) (layer "Edge.Cuts"))
 (gr_arc (start 172.02675 39.6375) (mid 173.708427 40.334073) (end 174.405 42.01575) (stroke (width 0.1) (type default)) (layer "Edge.Cuts"))
 (segment (start 116.3835 57.7135) (end 118.54225 59.87225) (width 0.254) (layer "B.Cu") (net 12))
 (segment (start 118.54225 59.87225) (end 119.40375 59.87225) (width 0.254) (layer "B.Cu") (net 12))
 (segment (start 123.91675 55.87225) (end 123.50375 56.28525) (width 0.381) (layer "B.Cu") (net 8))
 (segment (start 126.68925 68.1765) (end 128.30375 66.562) (width 0.381) (layer "B.Cu") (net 8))
 (segment (start 124.46825 68.97575) (end 121.90375 66.41125) (width 0.381) (layer "B.Cu") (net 8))
 (segment (start 124.386375 47.489625) (end 123.50375 48.37225) (width 0.381) (layer "B.Cu") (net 8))
 (segment (start 129.47475 48.99325) (end 129.37475 49.09325) (width 0.381) (layer "B.Cu") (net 8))
 (segment (start 129.21825 48.35775) (end 128.350125 47.489625) (width 0.381) (layer "B.Cu") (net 8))
 (segment (start 128.30375 66.562) (end 128.30375 65.57225) (width 0.381) (layer "B.Cu") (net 8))
 (segment (start 110.985 54.69975) (end 115.89875 59.6135) (width 0.381) (layer "B.Cu") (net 8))
 (segment (start 125.632 40.9585) (end 125.8965 41.223) (width 0.381) (layer "B.Cu") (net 8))
 (segment (start 127.07475 50.89325) (end 127.17475 50.79325) (width 0.381) (layer "B.Cu") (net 8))
 (segment (start 129.12475 49.09325) (end 129.37475 49.09325) (width 0.381) (layer "B.Cu") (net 8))
 (segment (start 121.90375 62.04125) (end 120.53475 60.67225) (width 0.381) (layer "B.Cu") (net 8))
 (segment (start 129.21825 48.93675) (end 129.21825 48.35775) (width 0.381) (layer "B.Cu") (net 8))
 (segment (start 110.985 47.527) (end 110.985 54.69975) (width 0.381) (layer "B.Cu") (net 8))
 (segment (start 124.24 40.9585) (end 125.632 40.9585) (width 0.381) (layer "B.Cu") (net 8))
 (segment (start 117.44225 60.67225) (end 119.40375 60.67225) (width 0.381) (layer "B.Cu") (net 8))
 (segment (start 125.10375 50.89325) (end 127.07475 50.89325) (width 0.381) (layer "B.Cu") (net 8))
 (segment (start 124.46825 69.762) (end 124.46825 72.14025) (width 0.381) (layer "B.Cu") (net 8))
 (segment (start 123.50375 54.17225) (end 123.50375 57.70325) (width 0.381) (layer "B.Cu") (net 8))
 (segment (start 120.53475 60.67225) (end 119.40375 60.67225) (width 0.381) (layer "B.Cu") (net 8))
 (segment (start 121.90375 65.57225) (end 121.90375 62.04125) (width 0.381) (layer "B.Cu") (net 8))
 (segment (start 115.89875 59.6135) (end 116.3835 59.6135) (width 0.381) (layer "B.Cu") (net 8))
 (segment (start 128.30375 64.44125) (end 128.30375 65.57225) (width 0.381) (layer "B.Cu") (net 8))
 (segment (start 123.50375 48.37225) (end 123.50375 54.17225) (width 0.381) (layer "B.Cu") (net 8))
 (segment (start 133.182 65.918) (end 131.2555 65.918) (width 0.381) (layer "B.Cu") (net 8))
 (segment (start 125.8965 45.9795) (end 124.386375 47.489625) (width 0.381) (layer "B.Cu") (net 8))
 (segment (start 127.17475 50.79325) (end 127.42475 50.79325) (width 0.381) (layer "B.Cu") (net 8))
 (segment (start 128.350125 47.489625) (end 124.386375 47.489625) (width 0.381) (layer "B.Cu") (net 8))
 (segment (start 126.68925 69.762) (end 126.68925 72.14025) (width 0.381) (layer "B.Cu") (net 8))
 (segment (start 130.80375 55.87225) (end 123.91675 55.87225) (width 0.381) (layer "B.Cu") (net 8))
 (segment (start 131.44575 48.99325) (end 129.47475 48.99325) (width 0.381) (layer "B.Cu") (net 8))
 (segment (start 116.3835 59.6135) (end 117.44225 60.67225) (width 0.381) (layer "B.Cu") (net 8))
 (segment (start 123.50375 57.70325) (end 120.53475 60.67225) (width 0.381) (layer "B.Cu") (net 8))
 (segment (start 128.31325 64.43175) (end 128.30375 64.44125) (width 0.381) (layer "B.Cu") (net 8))
 (segment (start 121.90375 66.41125) (end 121.90375 65.57225) (width 0.381) (layer "B.Cu") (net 8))
 (segment (start 131.2555 65.918) (end 129.76925 64.43175) (width 0.381) (layer "B.Cu") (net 8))
 (segment (start 124.46825 69.762) (end 124.46825 68.97575) (width 0.381) (layer "B.Cu") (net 8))
 (segment (start 124.46825 72.14025) (end 126.68925 72.14025) (width 0.381) (layer "B.Cu") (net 8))
 (segment (start 110.056 45.723) (end 110.056 46.598) (width 0.381) (layer "B.Cu") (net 8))
 (segment (start 110.056 46.598) (end 110.985 47.527) (width 0.381) (layer "B.Cu") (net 8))
 (segment (start 125.8965 41.223) (end 125.8965 45.9795) (width 0.381) (layer "B.Cu") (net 8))
 (segment (start 129.76925 64.43175) (end 128.31325 64.43175) (width 0.381) (layer "B.Cu") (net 8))
 (segment (start 129.37475 49.09325) (end 129.21825 48.93675) (width 0.381) (layer "B.Cu") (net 8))
 (segment (start 126.68925 69.762) (end 126.68925 68.1765) (width 0.381) (layer "B.Cu") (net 8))
 (segment (start 127.42475 50.79325) (end 129.12475 49.09325) (width 0.381) (layer "B.Cu") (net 8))
 (segment (start 116.8285 63.07225) (end 116.8285 52.82) (width 0.381) (layer "F.Cu") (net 9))
 (segment (start 116.8285 52.82) (end 117.327 52.3215) (width 0.381) (layer "F.Cu") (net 9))
 (segment (start 117.327 52.3215) (end 120.498 52.3215) (width 0.381) (layer "F.Cu") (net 9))
 (segment (start 120.44825 50.78575) (end 120.498 50.8355) (width 0.381) (layer "F.Cu") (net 9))
 (segment (start 120.498 50.8355) (end 120.498 52.3215) (width 0.381) (layer "F.Cu") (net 9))
 (segment (start 132.38925 52.3215) (end 133.182 53.11425) (width 0.381) (layer "F.Cu") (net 9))
 (segment (start 133.182 53.11425) (end 133.182 56.28525) (width 0.381) (layer "F.Cu") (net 9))
 (segment (start 120.498 52.3215) (end 132.38925 52.3215) (width 0.381) (layer "F.Cu") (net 9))
 (via (at 116.8285 63.07225) (size 0.8) (drill 0.4) (layers "F.Cu" "B.Cu") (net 9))
 (via (at 133.182 56.28525) (size 0.8) (drill 0.4) (layers "F.Cu" "B.Cu") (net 9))
 (via (at 120.44825 50.78575) (size 0.8) (drill 0.4) (layers "F.Cu" "B.Cu") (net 9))
 (segment (start 117.969 48.4775) (end 118.14 48.4775) (width 0.381) (layer "B.Cu") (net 9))
 (segment (start 122.56825 72.14025) (end 123.68375 73.25575) (width 0.381) (layer "B.Cu") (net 9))
 (segment (start 121.10375 68.2975) (end 121.10375 65.57225) (width 0.381) (layer "B.Cu") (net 9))
 (segment (start 121.10375 63.64125) (end 120.53475 63.07225) (width 0.381) (layer "B.Cu") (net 9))
 (segment (start 120.53475 63.07225) (end 119.40375 63.07225) (width 0.381) (layer "B.Cu") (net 9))
 (segment (start 132.795 56.67225) (end 130.80375 56.67225) (width 0.381) (layer "B.Cu") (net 9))
 (segment (start 116.8285 63.07225) (end 119.40375 63.07225) (width 0.381) (layer "B.Cu") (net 9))
 (segment (start 122.70375 56.90325) (end 122.70375 54.17225) (width 0.381) (layer "B.Cu") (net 9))
 (segment (start 122.56825 69.762) (end 121.10375 68.2975) (width 0.381) (layer "B.Cu") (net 9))
 (segment (start 107.66325 53.907) (end 116.8285 63.07225) (width 0.381) (layer "B.Cu") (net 9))
 (segment (start 122.70375 53.04125) (end 122.70375 54.17225) (width 0.381) (layer "B.Cu") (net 9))
 (segment (start 120.53475 59.07225) (end 122.70375 56.90325) (width 0.381) (layer "B.Cu") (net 9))
 (segment (start 103.6995 53.11425) (end 104.49225 53.907) (width 0.381) (layer "B.Cu") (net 9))
 (segment (start 127.47375 73.25575) (end 128.58925 72.14025) (width 0.381) (layer "B.Cu") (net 9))
 (segment (start 122.56825 69.762) (end 122.56825 72.14025) (width 0.381) (layer "B.Cu") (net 9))
 (segment (start 119.40375 59.07225) (end 120.53475 59.07225) (width 0.381) (layer "B.Cu") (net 9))
 (segment (start 104.49225 53.907) (end 107.66325 53.907) (width 0.381) (layer "B.Cu") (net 9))
 (segment (start 128.58925 69.762) (end 128.58925 72.14025) (width 0.381) (layer "B.Cu") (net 9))
 (segment (start 118.14 48.4775) (end 122.70375 53.04125) (width 0.381) (layer "B.Cu") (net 9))
 (segment (start 129.10375 69.2475) (end 129.10375 65.57225) (width 0.381) (layer "B.Cu") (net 9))
 (segment (start 133.182 56.28525) (end 132.795 56.67225) (width 0.381) (layer "B.Cu") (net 9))
 (segment (start 103.6995 52.3215) (end 103.6995 53.11425) (width 0.381) (layer "B.Cu") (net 9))
 (segment (start 123.68375 73.25575) (end 127.47375 73.25575) (width 0.381) (layer "B.Cu") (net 9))
 (segment (start 121.10375 65.57225) (end 121.10375 63.64125) (width 0.381) (layer "B.Cu") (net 9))
 (segment (start 128.58925 69.762) (end 129.10375 69.2475) (width 0.381) (layer "B.Cu") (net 9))
 (segment (start 125.20375 49.09325) (end 125.10375 48.99325) (width 0.254) (layer "B.Cu") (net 23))
 (segment (start 124.30375 53.107) (end 124.30375 54.17225) (width 0.254) (layer "B.Cu") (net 23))
 (segment (start 125.10375 48.99325) (end 124.05175 50.04525) (width 0.254) (layer "B.Cu") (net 23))
 (segment (start 127.17475 49.09325) (end 125.20375 49.09325) (width 0.254) (layer "B.Cu") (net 23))
 (segment (start 124.05175 50.04525) (end 124.05175 52.855) (width 0.254) (layer "B.Cu") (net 23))
 (segment (start 124.05175 52.855) (end 124.30375 53.107) (width 0.254) (layer "B.Cu") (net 23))
 (segment (start 129.37475 50.79325) (end 129.27475 50.79325) (width 0.254) (layer "B.Cu") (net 24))
 (segment (start 129.27475 50.79325) (end 127.482 52.586) (width 0.254) (layer "B.Cu") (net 24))
 (segment (start 125.10375 53.29325) (end 125.10375 54.17225) (width 0.254) (layer "B.Cu") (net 24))
 (segment (start 125.811 52.586) (end 125.10375 53.29325) (width 0.254) (layer "B.Cu") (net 24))
 (segment (start 129.37475 50.79325) (end 131.34575 50.79325) (width 0.254) (layer "B.Cu") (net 24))
 (segment (start 127.482 52.586) (end 125.811 52.586) (width 0.254) (layer "B.Cu") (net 24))
 (segment (start 131.34575 50.79325) (end 131.44575 50.89325) (width 0.254) (layer "B.Cu") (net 24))
 (segment (start 153.7935 57.078) (end 153.7935 50.8005) (width 0.254) (layer "B.Cu") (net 30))
 (segment (start 130.80375 57.47225) (end 153.39925 57.47225) (width 0.254) (layer "B.Cu") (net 30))
 (segment (start 154.5144 51.5214) (end 172.0341 51.5214) (width 0.254) (layer "B.Cu") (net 30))
 (segment (start 172.0341 51.5214) (end 172.8195 50.736) (width 0.254) (layer "B.Cu") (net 30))
 (segment (start 153.39925 57.47225) (end 153.7935 57.078) (width 0.254) (layer "B.Cu") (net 30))
 (segment (start 153.7935 50.8005) (end 154.5144 51.5214) (width 0.254) (layer "B.Cu") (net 30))
 (segment (start 148.366 44.6505) (end 150.9435 44.6505) (width 0.254) (layer "B.Cu") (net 6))
 (segment (start 150.9435 44.6505) (end 153.7935 47.5005) (width 0.254) (layer "B.Cu") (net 6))
 (segment (start 148.406 44.0705) (end 148.406 44.6105) (width 0.254) (layer "B.Cu") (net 6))
 (segment (start 148.406 44.6105) (end 148.366 44.6505) (width 0.254) (layer "B.Cu") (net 6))
 (segment (start 170.034 44.6505) (end 172.8195 47.436) (width 0.254) (layer "B.Cu") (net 3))
 (segment (start 167.392 44.1105) (end 167.432 44.0705) (width 0.254) (layer "B.Cu") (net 3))
 (segment (start 167.392 44.6505) (end 167.392 44.1105) (width 0.254) (layer "B.Cu") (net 3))
 (segment (start 167.392 44.6505) (end 170.034 44.6505) (width 0.254) (layer "B.Cu") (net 3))
 (segment (start 130.80375 59.07225) (end 154.995 59.07225) (width 0.254) (layer "B.Cu") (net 14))
 (segment (start 155.379 70.5474) (end 172.1631 70.5474) (width 0.254) (layer "B.Cu") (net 14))
 (segment (start 153.7935 69.891) (end 154.4499 70.5474) (width 0.254) (layer "B.Cu") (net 14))
 (segment (start 154.4499 70.5474) (end 155.379 70.5474) (width 0.254) (layer "B.Cu") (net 14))
 (segment (start 155.379 59.45625) (end 155.379 70.5474) (width 0.254) (layer "B.Cu") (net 14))
 (segment (start 172.1631 70.5474) (end 172.8195 69.891) (width 0.254) (layer "B.Cu") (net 14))
 (segment (start 154.995 59.07225) (end 155.379 59.45625) (width 0.254) (layer "B.Cu") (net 14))
 (segment (start 148.366 63.6765) (end 150.879 63.6765) (width 0.254) (layer "B.Cu") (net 5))
 (segment (start 150.879 63.6765) (end 153.7935 66.591) (width 0.254) (layer "B.Cu") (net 5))
 (segment (start 167.392 63.6765) (end 167.392 63.1365) (width 0.254) (layer "B.Cu") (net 2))
 (segment (start 169.905 63.6765) (end 172.8195 66.591) (width 0.254) (layer "B.Cu") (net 2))
 (segment (start 167.392 63.1365) (end 167.432 63.0965) (width 0.254) (layer "B.Cu") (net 2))
 (segment (start 167.392 63.6765) (end 169.905 63.6765) (width 0.254) (layer "B.Cu") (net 2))
 (segment (start 106.856 46.365) (end 106.856 45.723) (width 0.381) (layer "B.Cu") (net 13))
 (segment (start 103.6995 49.5215) (end 106.856 46.365) (width 0.381) (layer "B.Cu") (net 13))
 (segment (start 143.366 64.1765) (end 143.366 45.1505) (width 0.254) (layer "F.Cu") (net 4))
 (segment (start 141.5255 59.87225) (end 141.90225 60.249) (width 0.254) (layer "B.Cu") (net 4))
 (segment (start 130.80375 59.87225) (end 141.5255 59.87225) (width 0.254) (layer "B.Cu") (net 4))
 (segment (start 141.90225 65.48275) (end 142.056 65.6365) (width 0.254) (layer "B.Cu") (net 4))
 (segment (start 141.90225 60.249) (end 141.90225 65.48275) (width 0.254) (layer "B.Cu") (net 4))
 (segment (start 161.082 65.4865) (end 162.392 64.1765) (width 0.254) (layer "F.Cu") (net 1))
 (segment (start 161.082 65.6365) (end 161.082 65.4865) (width 0.254) (layer "F.Cu") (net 1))
 (segment (start 162.392 64.1765) (end 162.392 45.1505) (width 0.254) (layer "F.Cu") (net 1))
 (segment (start 161.082 58.81725) (end 161.082 65.6365) (width 0.254) (layer "B.Cu") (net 1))
 (segment (start 130.80375 58.27225) (end 160.537 58.27225) (width 0.254) (layer "B.Cu") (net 1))
 (segment (start 160.537 58.27225) (end 161.082 58.81725) (width 0.254) (layer "B.Cu") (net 1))
 (segment (start 131.0245 64.093) (end 130.80375 63.87225) (width 0.254) (layer "B.Cu") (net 7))
 (segment (start 133.182 64.093) (end 131.0245 64.093) (width 0.254) (layer "B.Cu") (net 7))
 (segment (start 108.456 49.03075) (end 109.24875 49.8235) (width 0.2) (layer "B.Cu") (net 43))
 (segment (start 108.456 45.723) (end 108.456 49.03075) (width 0.2) (layer "B.Cu") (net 43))
 (segment (start 116.701249 61.47225) (end 119.40375 61.47225) (width 0.254) (layer "B.Cu") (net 16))
 (segment (start 109.24875 51.6485) (end 109.24875 54.019751) (width 0.254) (layer "B.Cu") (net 16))
 (segment (start 109.24875 54.019751) (end 116.701249 61.47225) (width 0.254) (layer "B.Cu") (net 16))
 (segment (start 107.656 49.038) (end 106.8705 49.8235) (width 0.2) (layer "B.Cu") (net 10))
 (segment (start 107.656 45.723) (end 107.656 49.038) (width 0.2) (layer "B.Cu") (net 10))
 (segment (start 116.859197 62.27225) (end 119.40375 62.27225) (width 0.254) (layer "B.Cu") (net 11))
 (segment (start 106.8705 51.6485) (end 106.8705 52.283553) (width 0.254) (layer "B.Cu") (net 11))
 (segment (start 106.8705 52.283553) (end 116.859197 62.27225) (width 0.254) (layer "B.Cu") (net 11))
 (segment (start 116.942 47.6795) (end 116.942 48.979001) (width 0.254) (layer "B.Cu") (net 22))
 (segment (start 120.624802 52.661803) (end 121.397303 52.661803) (width 0.254) (layer "B.Cu") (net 22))
 (segment (start 116.942 48.979001) (end 120.624802 52.661803) (width 0.254) (layer "B.Cu") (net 22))
 (segment (start 121.90375 53.16825) (end 121.90375 54.17225) (width 0.254) (layer "B.Cu") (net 22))
 (segment (start 117.969 46.6525) (end 117.969 44.7295) (width 0.254) (layer "B.Cu") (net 22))
 (segment (start 117.969 44.7295) (end 118.04 44.6585) (width 0.254) (layer "B.Cu") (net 22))
 (segment (start 117.969 46.6525) (end 116.942 47.6795) (width 0.254) (layer "B.Cu") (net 22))
 (segment (start 121.397303 52.661803) (end 121.90375 53.16825) (width 0.254) (layer "B.Cu") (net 22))
 (segment (start 104.806 41.223) (end 104.806 45.723) (width 0.254) (layer "F.Cu") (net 44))
 (segment (start 104.806 41.223) (end 112.106 41.223) (width 0.254) (layer "F.Cu") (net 44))
 (segment (start 112.106 41.223) (end 112.106 45.723) (width 0.254) (layer "F.Cu") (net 44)))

